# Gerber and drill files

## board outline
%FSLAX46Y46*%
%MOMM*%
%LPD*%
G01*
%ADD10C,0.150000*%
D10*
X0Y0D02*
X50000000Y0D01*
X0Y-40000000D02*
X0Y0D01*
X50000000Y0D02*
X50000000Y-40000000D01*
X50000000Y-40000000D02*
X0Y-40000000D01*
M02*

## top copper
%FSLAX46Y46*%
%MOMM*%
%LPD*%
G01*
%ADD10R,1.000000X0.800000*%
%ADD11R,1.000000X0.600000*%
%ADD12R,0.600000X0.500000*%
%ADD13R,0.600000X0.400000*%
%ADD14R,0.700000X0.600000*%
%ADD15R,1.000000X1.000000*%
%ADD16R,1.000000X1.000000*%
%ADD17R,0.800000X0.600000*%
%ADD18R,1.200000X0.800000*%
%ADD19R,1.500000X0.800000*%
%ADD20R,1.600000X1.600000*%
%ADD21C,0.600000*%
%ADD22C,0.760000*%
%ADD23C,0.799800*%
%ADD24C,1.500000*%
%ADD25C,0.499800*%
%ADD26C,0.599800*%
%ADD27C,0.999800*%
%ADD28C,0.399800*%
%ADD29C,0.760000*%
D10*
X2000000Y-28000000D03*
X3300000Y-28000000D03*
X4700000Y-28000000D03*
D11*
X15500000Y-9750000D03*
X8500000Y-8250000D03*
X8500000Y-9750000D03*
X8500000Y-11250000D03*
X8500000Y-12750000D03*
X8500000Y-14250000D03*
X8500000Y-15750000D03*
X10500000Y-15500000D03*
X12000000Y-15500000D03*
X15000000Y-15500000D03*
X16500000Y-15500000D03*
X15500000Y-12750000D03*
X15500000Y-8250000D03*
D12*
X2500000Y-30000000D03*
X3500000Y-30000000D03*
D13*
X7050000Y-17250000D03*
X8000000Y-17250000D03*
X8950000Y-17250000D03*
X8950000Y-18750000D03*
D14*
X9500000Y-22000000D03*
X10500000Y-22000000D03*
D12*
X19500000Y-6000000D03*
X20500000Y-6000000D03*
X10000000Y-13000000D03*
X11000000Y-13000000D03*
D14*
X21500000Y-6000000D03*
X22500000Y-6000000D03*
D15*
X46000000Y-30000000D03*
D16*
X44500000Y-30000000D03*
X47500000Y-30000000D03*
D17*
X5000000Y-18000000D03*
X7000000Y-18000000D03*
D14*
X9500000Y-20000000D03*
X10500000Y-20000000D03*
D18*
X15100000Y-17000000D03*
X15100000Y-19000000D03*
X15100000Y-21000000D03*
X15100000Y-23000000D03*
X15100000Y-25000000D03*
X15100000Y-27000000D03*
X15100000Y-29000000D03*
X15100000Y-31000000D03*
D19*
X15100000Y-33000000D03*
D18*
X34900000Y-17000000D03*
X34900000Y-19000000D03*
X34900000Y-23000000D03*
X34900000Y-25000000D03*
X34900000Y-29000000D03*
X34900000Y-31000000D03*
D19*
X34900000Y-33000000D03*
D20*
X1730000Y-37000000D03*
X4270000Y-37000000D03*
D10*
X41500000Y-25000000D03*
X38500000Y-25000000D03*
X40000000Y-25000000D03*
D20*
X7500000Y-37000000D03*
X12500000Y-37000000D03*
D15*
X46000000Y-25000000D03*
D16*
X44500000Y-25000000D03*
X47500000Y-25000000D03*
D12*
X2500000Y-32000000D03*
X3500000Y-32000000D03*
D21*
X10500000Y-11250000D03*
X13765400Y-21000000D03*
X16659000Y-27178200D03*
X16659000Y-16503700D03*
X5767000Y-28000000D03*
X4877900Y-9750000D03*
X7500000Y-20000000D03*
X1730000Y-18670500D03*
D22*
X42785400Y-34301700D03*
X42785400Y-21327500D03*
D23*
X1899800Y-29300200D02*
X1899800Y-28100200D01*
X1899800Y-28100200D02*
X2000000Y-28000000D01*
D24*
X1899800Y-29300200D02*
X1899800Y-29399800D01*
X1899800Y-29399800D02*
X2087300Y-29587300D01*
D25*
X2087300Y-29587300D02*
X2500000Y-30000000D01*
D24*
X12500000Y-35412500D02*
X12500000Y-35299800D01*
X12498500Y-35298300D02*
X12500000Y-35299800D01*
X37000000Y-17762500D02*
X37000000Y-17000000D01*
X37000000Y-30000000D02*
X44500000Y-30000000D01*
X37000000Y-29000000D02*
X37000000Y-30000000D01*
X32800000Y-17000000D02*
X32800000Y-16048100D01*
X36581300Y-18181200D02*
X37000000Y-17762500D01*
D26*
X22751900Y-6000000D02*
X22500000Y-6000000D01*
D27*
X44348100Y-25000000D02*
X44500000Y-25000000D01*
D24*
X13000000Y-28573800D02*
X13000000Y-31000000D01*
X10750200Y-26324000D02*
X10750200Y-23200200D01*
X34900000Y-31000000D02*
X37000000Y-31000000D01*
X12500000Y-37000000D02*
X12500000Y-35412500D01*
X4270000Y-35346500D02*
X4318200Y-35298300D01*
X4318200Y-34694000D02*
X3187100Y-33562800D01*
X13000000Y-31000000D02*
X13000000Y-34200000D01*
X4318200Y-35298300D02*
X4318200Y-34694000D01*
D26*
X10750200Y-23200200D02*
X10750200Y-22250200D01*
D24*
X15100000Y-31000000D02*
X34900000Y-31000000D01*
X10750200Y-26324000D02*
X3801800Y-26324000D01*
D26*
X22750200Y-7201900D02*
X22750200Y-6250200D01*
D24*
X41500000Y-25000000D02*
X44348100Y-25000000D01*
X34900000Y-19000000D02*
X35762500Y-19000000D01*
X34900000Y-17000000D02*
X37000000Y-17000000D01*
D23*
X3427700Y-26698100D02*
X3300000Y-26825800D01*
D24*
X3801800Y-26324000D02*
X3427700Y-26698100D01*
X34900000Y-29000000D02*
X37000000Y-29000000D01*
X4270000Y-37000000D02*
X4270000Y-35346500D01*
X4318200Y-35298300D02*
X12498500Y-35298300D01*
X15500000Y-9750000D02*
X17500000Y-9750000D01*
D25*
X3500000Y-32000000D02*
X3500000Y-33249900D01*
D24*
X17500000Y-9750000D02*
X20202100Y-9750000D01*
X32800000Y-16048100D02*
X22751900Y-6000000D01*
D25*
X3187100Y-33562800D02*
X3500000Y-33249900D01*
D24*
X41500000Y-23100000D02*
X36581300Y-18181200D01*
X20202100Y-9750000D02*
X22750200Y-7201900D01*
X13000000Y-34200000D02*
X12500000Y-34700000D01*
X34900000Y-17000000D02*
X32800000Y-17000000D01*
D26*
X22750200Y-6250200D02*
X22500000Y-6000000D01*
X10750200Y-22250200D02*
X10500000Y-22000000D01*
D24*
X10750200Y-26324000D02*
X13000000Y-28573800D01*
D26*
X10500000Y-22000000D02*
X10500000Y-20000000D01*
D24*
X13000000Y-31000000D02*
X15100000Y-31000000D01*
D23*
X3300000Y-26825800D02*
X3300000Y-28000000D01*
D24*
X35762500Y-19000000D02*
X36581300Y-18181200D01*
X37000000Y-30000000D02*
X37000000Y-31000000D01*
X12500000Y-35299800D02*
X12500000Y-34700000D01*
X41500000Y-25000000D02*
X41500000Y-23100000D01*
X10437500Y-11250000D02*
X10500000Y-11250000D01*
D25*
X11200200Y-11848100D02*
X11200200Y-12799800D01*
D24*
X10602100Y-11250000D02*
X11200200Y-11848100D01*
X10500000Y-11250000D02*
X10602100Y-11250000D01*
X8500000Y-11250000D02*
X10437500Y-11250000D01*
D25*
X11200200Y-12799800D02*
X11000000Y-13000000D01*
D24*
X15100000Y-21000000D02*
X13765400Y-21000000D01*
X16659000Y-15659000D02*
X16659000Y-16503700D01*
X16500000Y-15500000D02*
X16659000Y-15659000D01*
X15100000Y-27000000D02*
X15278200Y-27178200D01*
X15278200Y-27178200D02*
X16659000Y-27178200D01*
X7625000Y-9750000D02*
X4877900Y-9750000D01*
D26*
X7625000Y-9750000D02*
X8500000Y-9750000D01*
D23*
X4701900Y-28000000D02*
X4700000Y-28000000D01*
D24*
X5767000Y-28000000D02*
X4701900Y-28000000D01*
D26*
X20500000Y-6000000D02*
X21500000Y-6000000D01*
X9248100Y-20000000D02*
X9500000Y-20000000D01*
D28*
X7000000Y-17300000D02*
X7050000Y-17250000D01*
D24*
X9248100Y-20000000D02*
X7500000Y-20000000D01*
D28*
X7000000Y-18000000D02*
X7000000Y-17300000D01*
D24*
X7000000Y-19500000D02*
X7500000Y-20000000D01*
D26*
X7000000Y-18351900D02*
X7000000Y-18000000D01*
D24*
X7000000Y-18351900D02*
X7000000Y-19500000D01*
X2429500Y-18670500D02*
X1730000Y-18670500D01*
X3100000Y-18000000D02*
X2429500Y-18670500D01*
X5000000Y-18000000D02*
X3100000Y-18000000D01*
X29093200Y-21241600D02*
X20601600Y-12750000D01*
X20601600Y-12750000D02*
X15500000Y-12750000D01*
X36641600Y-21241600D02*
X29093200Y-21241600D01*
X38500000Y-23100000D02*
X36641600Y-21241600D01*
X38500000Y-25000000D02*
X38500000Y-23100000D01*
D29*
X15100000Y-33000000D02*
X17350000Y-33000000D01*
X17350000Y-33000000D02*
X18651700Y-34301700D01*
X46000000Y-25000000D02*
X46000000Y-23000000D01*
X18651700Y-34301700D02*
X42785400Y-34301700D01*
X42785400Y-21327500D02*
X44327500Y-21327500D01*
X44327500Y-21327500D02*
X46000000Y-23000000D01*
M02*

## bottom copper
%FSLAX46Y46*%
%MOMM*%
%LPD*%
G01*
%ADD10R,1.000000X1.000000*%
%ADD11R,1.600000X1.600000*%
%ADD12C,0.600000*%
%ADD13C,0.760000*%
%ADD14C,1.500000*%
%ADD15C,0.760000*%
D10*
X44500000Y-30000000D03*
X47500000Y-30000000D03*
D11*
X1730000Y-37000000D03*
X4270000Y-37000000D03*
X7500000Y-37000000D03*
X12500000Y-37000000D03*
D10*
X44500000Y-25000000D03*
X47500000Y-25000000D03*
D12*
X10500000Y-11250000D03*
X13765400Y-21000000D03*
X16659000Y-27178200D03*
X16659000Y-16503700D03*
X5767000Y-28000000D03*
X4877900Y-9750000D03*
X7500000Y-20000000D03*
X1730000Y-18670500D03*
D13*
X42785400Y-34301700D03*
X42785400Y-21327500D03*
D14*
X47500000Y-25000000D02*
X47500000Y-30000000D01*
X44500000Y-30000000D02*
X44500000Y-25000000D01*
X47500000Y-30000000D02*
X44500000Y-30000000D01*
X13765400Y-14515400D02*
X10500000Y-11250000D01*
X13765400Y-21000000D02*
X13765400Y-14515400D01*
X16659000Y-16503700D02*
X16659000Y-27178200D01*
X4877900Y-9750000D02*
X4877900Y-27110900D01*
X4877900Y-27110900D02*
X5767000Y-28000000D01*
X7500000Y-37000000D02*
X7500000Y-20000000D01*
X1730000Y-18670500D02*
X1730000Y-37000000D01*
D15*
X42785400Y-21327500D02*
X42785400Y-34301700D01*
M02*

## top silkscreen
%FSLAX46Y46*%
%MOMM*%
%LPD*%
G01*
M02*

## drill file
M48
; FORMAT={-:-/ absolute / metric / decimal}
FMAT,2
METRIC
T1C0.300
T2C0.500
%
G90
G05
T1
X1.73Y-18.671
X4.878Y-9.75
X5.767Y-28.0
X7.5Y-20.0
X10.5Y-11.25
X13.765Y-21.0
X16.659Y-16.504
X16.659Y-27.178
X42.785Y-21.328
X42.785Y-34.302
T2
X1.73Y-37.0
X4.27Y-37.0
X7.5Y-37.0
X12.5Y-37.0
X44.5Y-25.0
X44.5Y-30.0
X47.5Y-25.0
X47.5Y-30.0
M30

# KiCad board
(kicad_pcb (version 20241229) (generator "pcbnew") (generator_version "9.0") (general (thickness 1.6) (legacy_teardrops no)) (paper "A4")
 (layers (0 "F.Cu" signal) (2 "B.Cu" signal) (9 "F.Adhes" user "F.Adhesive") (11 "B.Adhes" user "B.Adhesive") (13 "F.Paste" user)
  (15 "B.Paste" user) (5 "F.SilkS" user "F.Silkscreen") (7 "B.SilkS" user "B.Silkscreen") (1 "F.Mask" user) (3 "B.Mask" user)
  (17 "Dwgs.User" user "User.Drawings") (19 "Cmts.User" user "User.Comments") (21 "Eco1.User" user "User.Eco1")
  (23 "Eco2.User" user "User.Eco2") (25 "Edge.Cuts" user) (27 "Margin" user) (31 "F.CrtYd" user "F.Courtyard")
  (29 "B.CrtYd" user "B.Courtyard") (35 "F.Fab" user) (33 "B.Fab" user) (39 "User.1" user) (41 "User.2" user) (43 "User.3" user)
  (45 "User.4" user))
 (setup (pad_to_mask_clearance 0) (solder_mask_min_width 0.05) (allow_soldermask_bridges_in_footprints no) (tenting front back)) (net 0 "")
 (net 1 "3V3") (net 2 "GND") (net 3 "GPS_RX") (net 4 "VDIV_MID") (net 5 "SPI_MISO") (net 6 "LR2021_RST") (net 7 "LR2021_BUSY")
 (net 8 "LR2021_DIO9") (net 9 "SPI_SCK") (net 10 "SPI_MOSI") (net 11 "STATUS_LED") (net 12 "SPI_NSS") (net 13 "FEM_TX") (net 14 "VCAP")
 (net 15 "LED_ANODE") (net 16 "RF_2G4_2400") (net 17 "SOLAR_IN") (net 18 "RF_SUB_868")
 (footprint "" (layer "F.Cu") (at 4 28)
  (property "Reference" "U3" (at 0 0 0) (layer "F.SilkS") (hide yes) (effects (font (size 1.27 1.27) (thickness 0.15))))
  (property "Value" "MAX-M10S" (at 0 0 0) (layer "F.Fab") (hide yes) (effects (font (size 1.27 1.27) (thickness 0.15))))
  (pad "1" smd rect (at -2 0) (size 1 0.8) (layers "F.Cu" "F.Mask") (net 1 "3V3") (thermal_bridge_angle 45))
  (pad "2" smd rect (at -0.7 0) (size 1 0.8) (layers "F.Cu" "F.Mask") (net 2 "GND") (thermal_bridge_angle 45))
  (pad "3" smd rect (at 0.7 0) (size 1 0.8) (layers "F.Cu" "F.Mask") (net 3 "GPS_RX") (thermal_bridge_angle 45)))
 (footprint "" (layer "F.Cu") (at 12 12)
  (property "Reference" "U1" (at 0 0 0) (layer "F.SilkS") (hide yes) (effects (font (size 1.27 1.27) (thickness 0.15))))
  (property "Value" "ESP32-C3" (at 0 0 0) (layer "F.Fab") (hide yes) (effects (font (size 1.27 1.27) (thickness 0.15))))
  (pad "GND" smd rect (at 3.5 -2.25) (size 1 0.6) (layers "F.Cu" "F.Mask") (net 2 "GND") (thermal_bridge_angle 45))
  (pad "GPIO0" smd rect (at -3.5 -3.75) (size 1 0.6) (layers "F.Cu" "F.Mask") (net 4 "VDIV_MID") (thermal_bridge_angle 45))
  (pad "GPIO1" smd rect (at -3.5 -2.25) (size 1 0.6) (layers "F.Cu" "F.Mask") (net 3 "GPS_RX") (thermal_bridge_angle 45))
  (pad "GPIO2" smd rect (at -3.5 -0.75) (size 1 0.6) (layers "F.Cu" "F.Mask") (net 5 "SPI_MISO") (thermal_bridge_angle 45))
  (pad "GPIO3" smd rect (at -3.5 0.75) (size 1 0.6) (layers "F.Cu" "F.Mask") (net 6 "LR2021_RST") (thermal_bridge_angle 45))
  (pad "GPIO4" smd rect (at -3.5 2.25) (size 1 0.6) (layers "F.Cu" "F.Mask") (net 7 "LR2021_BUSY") (thermal_bridge_angle 45))
  (pad "GPIO5" smd rect (at -3.5 3.75) (size 1 0.6) (layers "F.Cu" "F.Mask") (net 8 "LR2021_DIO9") (thermal_bridge_angle 45))
  (pad "GPIO6" smd rect (at -1.5 3.5) (size 1 0.6) (layers "F.Cu" "F.Mask") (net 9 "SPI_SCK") (thermal_bridge_angle 45))
  (pad "GPIO7" smd rect (at 0 3.5) (size 1 0.6) (layers "F.Cu" "F.Mask") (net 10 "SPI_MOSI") (thermal_bridge_angle 45))
  (pad "GPIO9" smd rect (at 3 3.5) (size 1 0.6) (layers "F.Cu" "F.Mask") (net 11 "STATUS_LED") (thermal_bridge_angle 45))
  (pad "GPIO10" smd rect (at 4.5 3.5) (size 1 0.6) (layers "F.Cu" "F.Mask") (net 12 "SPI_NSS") (thermal_bridge_angle 45))
  (pad "GPIO19" smd rect (at 3.5 0.75) (size 1 0.6) (layers "F.Cu" "F.Mask") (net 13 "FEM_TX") (thermal_bridge_angle 45))
  (pad "VCC" smd rect (at 3.5 -3.75) (size 1 0.6) (layers "F.Cu" "F.Mask") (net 1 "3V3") (thermal_bridge_angle 45)))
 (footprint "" (layer "F.Cu") (at 3 30)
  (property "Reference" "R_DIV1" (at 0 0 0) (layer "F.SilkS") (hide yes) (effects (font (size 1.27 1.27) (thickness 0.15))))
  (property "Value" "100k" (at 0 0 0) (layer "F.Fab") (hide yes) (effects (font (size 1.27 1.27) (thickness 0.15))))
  (pad "1" smd rect (at -0.5 0) (size 0.6 0.5) (layers "F.Cu" "F.Mask") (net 1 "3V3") (thermal_bridge_angle 45))
  (pad "2" smd rect (at 0.5 0) (size 0.6 0.5) (layers "F.Cu" "F.Mask") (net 4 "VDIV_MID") (thermal_bridge_angle 45)))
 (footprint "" (layer "F.Cu") (at 8 18)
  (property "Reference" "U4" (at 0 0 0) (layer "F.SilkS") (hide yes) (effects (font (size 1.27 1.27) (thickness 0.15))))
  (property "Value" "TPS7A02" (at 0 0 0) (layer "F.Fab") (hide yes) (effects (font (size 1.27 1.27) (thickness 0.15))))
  (pad "1" smd rect (at -0.95 -0.75) (size 0.6 0.4) (layers "F.Cu" "F.Mask") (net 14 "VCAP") (thermal_bridge_angle 45))
  (pad "2" smd rect (at 0 -0.75) (size 0.6 0.4) (layers "F.Cu" "F.Mask") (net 2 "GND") (thermal_bridge_angle 45))
  (pad "3" smd rect (at 0.95 -0.75) (size 0.6 0.4) (layers "F.Cu" "F.Mask") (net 14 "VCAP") (thermal_bridge_angle 45))
  (pad "4" smd rect (at 0.95 0.75) (size 0.6 0.4) (layers "F.Cu" "F.Mask") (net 1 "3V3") (thermal_bridge_angle 45)))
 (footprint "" (layer "F.Cu") (at 10 22)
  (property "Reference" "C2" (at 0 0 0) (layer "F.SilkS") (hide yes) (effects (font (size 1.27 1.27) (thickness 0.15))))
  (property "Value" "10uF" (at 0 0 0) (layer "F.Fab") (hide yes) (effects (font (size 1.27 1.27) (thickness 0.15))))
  (pad "1" smd rect (at -0.5 0) (size 0.7 0.6) (layers "F.Cu" "F.Mask") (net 1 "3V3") (thermal_bridge_angle 45))
  (pad "2" smd rect (at 0.5 0) (size 0.7 0.6) (layers "F.Cu" "F.Mask") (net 2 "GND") (thermal_bridge_angle 45)))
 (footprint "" (layer "F.Cu") (at 20 6)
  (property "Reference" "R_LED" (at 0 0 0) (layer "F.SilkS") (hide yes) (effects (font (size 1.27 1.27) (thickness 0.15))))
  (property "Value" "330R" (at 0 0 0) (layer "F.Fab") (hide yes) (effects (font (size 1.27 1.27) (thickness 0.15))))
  (pad "1" smd rect (at -0.5 0) (size 0.6 0.5) (layers "F.Cu" "F.Mask") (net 11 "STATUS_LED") (thermal_bridge_angle 45))
  (pad "2" smd rect (at 0.5 0) (size 0.6 0.5) (layers "F.Cu" "F.Mask") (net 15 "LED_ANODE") (thermal_bridge_angle 45)))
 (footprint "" (layer "F.Cu") (at 10.5 13)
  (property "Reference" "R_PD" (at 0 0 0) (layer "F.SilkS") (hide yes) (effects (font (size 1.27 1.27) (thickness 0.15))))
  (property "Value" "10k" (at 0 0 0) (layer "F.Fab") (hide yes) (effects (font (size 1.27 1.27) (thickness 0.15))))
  (pad "1" smd rect (at -0.5 0) (size 0.6 0.5) (layers "F.Cu" "F.Mask") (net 2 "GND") (thermal_bridge_angle 45))
  (pad "2" smd rect (at 0.5 0) (size 0.6 0.5) (layers "F.Cu" "F.Mask") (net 5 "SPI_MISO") (thermal_bridge_angle 45)))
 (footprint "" (layer "F.Cu") (at 22 6)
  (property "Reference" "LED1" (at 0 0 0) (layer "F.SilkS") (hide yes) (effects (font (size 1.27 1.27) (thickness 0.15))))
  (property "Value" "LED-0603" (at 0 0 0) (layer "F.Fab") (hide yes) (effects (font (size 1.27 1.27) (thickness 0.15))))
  (pad "A" smd rect (at -0.5 0) (size 0.7 0.6) (layers "F.Cu" "F.Mask") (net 15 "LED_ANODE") (thermal_bridge_angle 45))
  (pad "K" smd rect (at 0.5 0) (size 0.7 0.6) (layers "F.Cu" "F.Mask") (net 2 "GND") (thermal_bridge_angle 45)))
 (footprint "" (layer "F.Cu") (at 46 30)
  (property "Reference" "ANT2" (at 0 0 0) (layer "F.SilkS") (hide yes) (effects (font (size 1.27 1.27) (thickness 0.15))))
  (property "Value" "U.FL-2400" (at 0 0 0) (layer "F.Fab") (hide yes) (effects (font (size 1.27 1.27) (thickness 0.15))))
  (pad "1" smd rect (at 0 0) (size 1 1) (layers "F.Cu" "F.Mask") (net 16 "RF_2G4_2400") (thermal_bridge_angle 45))
  (pad "2" thru_hole rect (at -1.5 0) (size 1 1) (drill 0.5) (layers "*.Cu" "*.Mask") (remove_unused_layers no) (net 2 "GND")
   (thermal_bridge_angle 45))
  (pad "3" thru_hole rect (at 1.5 0) (size 1 1) (drill 0.5) (layers "*.Cu" "*.Mask") (remove_unused_layers no) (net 2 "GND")
   (thermal_bridge_angle 45)))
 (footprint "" (layer "F.Cu") (at 6 18)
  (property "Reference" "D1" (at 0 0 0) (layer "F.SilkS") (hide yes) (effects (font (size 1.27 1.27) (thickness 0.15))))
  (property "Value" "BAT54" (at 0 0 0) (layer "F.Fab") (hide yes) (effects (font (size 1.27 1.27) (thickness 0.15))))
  (pad "A" smd rect (at -1 0) (size 0.8 0.6) (layers "F.Cu" "F.Mask") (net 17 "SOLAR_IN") (thermal_bridge_angle 45))
  (pad "K" smd rect (at 1 0) (size 0.8 0.6) (layers "F.Cu" "F.Mask") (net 14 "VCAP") (thermal_bridge_angle 45)))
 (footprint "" (layer "F.Cu") (at 10 20)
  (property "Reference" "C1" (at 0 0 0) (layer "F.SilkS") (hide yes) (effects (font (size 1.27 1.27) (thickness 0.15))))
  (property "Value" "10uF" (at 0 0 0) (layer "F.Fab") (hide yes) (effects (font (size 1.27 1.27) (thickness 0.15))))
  (pad "1" smd rect (at -0.5 0) (size 0.7 0.6) (layers "F.Cu" "F.Mask") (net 14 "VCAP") (thermal_bridge_angle 45))
  (pad "2" smd rect (at 0.5 0) (size 0.7 0.6) (layers "F.Cu" "F.Mask") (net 2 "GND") (thermal_bridge_angle 45)))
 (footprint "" (layer "F.Cu") (at 25 25)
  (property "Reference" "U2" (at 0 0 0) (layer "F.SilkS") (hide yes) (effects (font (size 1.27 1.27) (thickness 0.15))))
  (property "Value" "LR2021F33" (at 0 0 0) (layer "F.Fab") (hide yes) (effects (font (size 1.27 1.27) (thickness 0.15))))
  (pad "1" smd rect (at -9.9 -8) (size 1.2 0.8) (layers "F.Cu" "F.Mask") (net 1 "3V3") (thermal_bridge_angle 45))
  (pad "2" smd rect (at -9.9 -6) (size 1.2 0.8) (layers "F.Cu" "F.Mask") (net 2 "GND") (thermal_bridge_angle 45))
  (pad "3" smd rect (at -9.9 -4) (size 1.2 0.8) (layers "F.Cu" "F.Mask") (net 5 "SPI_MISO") (thermal_bridge_angle 45))
  (pad "4" smd rect (at -9.9 -2) (size 1.2 0.8) (layers "F.Cu" "F.Mask") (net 10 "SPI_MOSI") (thermal_bridge_angle 45))
  (pad "5" smd rect (at -9.9 0) (size 1.2 0.8) (layers "F.Cu" "F.Mask") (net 9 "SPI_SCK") (thermal_bridge_angle 45))
  (pad "6" smd rect (at -9.9 2) (size 1.2 0.8) (layers "F.Cu" "F.Mask") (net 12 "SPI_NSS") (thermal_bridge_angle 45))
  (pad "7" smd rect (at -9.9 4) (size 1.2 0.8) (layers "F.Cu" "F.Mask") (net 7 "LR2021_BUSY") (thermal_bridge_angle 45))
  (pad "8" smd rect (at -9.9 6) (size 1.2 0.8) (layers "F.Cu" "F.Mask") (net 2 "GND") (thermal_bridge_angle 45))
  (pad "9" smd rect (at -9.9 8) (size 1.5 0.8) (layers "F.Cu" "F.Mask") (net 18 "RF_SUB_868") (thermal_bridge_angle 45))
  (pad "10" smd rect (at 9.9 -8) (size 1.2 0.8) (layers "F.Cu" "F.Mask") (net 2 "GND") (thermal_bridge_angle 45))
  (pad "11" smd rect (at 9.9 -6) (size 1.2 0.8) (layers "F.Cu" "F.Mask") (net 2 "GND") (thermal_bridge_angle 45))
  (pad "13" smd rect (at 9.9 -2) (size 1.2 0.8) (layers "F.Cu" "F.Mask") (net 8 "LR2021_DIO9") (thermal_bridge_angle 45))
  (pad "14" smd rect (at 9.9 0) (size 1.2 0.8) (layers "F.Cu" "F.Mask") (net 6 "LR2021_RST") (thermal_bridge_angle 45))
  (pad "16" smd rect (at 9.9 4) (size 1.2 0.8) (layers "F.Cu" "F.Mask") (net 2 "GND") (thermal_bridge_angle 45))
  (pad "17" smd rect (at 9.9 6) (size 1.2 0.8) (layers "F.Cu" "F.Mask") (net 2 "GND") (thermal_bridge_angle 45))
  (pad "18" smd rect (at 9.9 8) (size 1.5 0.8) (layers "F.Cu" "F.Mask") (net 16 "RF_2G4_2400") (thermal_bridge_angle 45)))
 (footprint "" (layer "F.Cu") (at 3 37)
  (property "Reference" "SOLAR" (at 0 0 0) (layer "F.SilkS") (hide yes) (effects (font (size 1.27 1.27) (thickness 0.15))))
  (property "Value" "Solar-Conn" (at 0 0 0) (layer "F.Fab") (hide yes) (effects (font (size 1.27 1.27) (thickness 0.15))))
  (pad "1" thru_hole rect (at -1.27 0) (size 1.6 1.6) (drill 0.5) (layers "*.Cu" "*.Mask") (remove_unused_layers no) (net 17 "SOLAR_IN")
   (thermal_bridge_angle 45))
  (pad "2" thru_hole rect (at 1.27 0) (size 1.6 1.6) (drill 0.5) (layers "*.Cu" "*.Mask") (remove_unused_layers no) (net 2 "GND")
   (thermal_bridge_angle 45)))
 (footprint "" (layer "F.Cu") (at 40 25)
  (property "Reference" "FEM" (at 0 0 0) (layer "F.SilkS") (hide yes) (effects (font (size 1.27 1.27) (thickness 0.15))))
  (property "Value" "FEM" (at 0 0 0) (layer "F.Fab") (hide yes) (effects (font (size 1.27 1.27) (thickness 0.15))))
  (pad "GND" smd rect (at 1.5 0) (size 1 0.8) (layers "F.Cu" "F.Mask") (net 2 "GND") (thermal_bridge_angle 45))
  (pad "TX" smd rect (at -1.5 0) (size 1 0.8) (layers "F.Cu" "F.Mask") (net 13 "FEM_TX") (thermal_bridge_angle 45))
  (pad "VCC" smd rect (at 0 0) (size 1 0.8) (layers "F.Cu" "F.Mask") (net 1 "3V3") (thermal_bridge_angle 45)))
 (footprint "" (layer "F.Cu") (at 10 37)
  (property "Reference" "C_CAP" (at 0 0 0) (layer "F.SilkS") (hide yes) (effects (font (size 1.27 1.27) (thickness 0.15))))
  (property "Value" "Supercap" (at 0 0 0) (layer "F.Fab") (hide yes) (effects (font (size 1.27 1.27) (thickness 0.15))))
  (pad "1" thru_hole rect (at -2.5 0) (size 1.6 1.6) (drill 0.5) (layers "*.Cu" "*.Mask") (remove_unused_layers no) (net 14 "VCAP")
   (thermal_bridge_angle 45))
  (pad "2" thru_hole rect (at 2.5 0) (size 1.6 1.6) (drill 0.5) (layers "*.Cu" "*.Mask") (remove_unused_layers no) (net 2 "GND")
   (thermal_bridge_angle 45)))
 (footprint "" (layer "F.Cu") (at 46 25)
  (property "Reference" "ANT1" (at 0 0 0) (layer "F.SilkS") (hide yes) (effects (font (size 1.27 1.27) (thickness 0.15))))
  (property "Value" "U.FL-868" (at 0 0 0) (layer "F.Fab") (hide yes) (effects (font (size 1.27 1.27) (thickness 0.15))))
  (pad "1" smd rect (at 0 0) (size 1 1) (layers "F.Cu" "F.Mask") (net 18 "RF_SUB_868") (thermal_bridge_angle 45))
  (pad "2" thru_hole rect (at -1.5 0) (size 1 1) (drill 0.5) (layers "*.Cu" "*.Mask") (remove_unused_layers no) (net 2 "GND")
   (thermal_bridge_angle 45))
  (pad "3" thru_hole rect (at 1.5 0) (size 1 1) (drill 0.5) (layers "*.Cu" "*.Mask") (remove_unused_layers no) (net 2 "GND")
   (thermal_bridge_angle 45)))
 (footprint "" (layer "F.Cu") (at 3 32)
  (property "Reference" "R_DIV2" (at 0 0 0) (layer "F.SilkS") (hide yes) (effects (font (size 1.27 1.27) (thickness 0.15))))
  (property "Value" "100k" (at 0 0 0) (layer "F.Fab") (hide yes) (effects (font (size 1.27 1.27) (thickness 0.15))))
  (pad "1" smd rect (at -0.5 0) (size 0.6 0.5) (layers "F.Cu" "F.Mask") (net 4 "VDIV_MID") (thermal_bridge_angle 45))
  (pad "2" smd rect (at 0.5 0) (size 0.6 0.5) (layers "F.Cu" "F.Mask") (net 2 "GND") (thermal_bridge_angle 45)))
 (gr_line (start 0 0) (end 50 0) (stroke (width 0.15) (type default)) (layer "Edge.Cuts"))
 (gr_line (start 0 40) (end 0 0) (stroke (width 0.15) (type default)) (layer "Edge.Cuts"))
 (gr_line (start 50 0) (end 50 40) (stroke (width 0.15) (type default)) (layer "Edge.Cuts"))
 (gr_line (start 50 40) (end 0 40) (stroke (width 0.15) (type default)) (layer "Edge.Cuts"))
 (segment (start 1.8998 29.3002) (end 1.8998 28.1002) (width 0.7998) (layer "F.Cu") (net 1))
 (segment (start 1.8998 28.1002) (end 2 28) (width 0.7998) (layer "F.Cu") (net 1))
 (segment (start 1.8998 29.3002) (end 1.8998 29.3998) (width 1.5) (layer "F.Cu") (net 1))
 (segment (start 1.8998 29.3998) (end 2.0873 29.5873) (width 1.5) (layer "F.Cu") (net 1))
 (segment (start 2.0873 29.5873) (end 2.5 30) (width 0.4998) (layer "F.Cu") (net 1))
 (segment (start 12.5 35.4125) (end 12.5 35.2998) (width 1.5) (layer "F.Cu") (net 2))
 (segment (start 12.4985 35.2983) (end 12.5 35.2998) (width 1.5) (layer "F.Cu") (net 2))
 (segment (start 37 17.7625) (end 37 17) (width 1.5) (layer "F.Cu") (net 2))
 (segment (start 37 30) (end 44.5 30) (width 1.5) (layer "F.Cu") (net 2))
 (segment (start 37 29) (end 37 30) (width 1.5) (layer "F.Cu") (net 2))
 (segment (start 32.8 17) (end 32.8 16.0481) (width 1.5) (layer "F.Cu") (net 2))
 (segment (start 36.5813 18.1812) (end 37 17.7625) (width 1.5) (layer "F.Cu") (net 2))
 (segment (start 22.7519 6) (end 22.5 6) (width 0.5998) (layer "F.Cu") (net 2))
 (segment (start 44.3481 25) (end 44.5 25) (width 0.9998) (layer "F.Cu") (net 2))
 (segment (start 13 28.5738) (end 13 31) (width 1.5) (layer "F.Cu") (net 2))
 (segment (start 10.7502 26.324) (end 10.7502 23.2002) (width 1.5) (layer "F.Cu") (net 2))
 (segment (start 34.9 31) (end 37 31) (width 1.5) (layer "F.Cu") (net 2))
 (segment (start 12.5 37) (end 12.5 35.4125) (width 1.5) (layer "F.Cu") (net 2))
 (segment (start 4.27 35.3465) (end 4.3182 35.2983) (width 1.5) (layer "F.Cu") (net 2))
 (segment (start 4.3182 34.694) (end 3.1871 33.5628) (width 1.5) (layer "F.Cu") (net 2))
 (segment (start 13 31) (end 13 34.2) (width 1.5) (layer "F.Cu") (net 2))
 (segment (start 4.3182 35.2983) (end 4.3182 34.694) (width 1.5) (layer "F.Cu") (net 2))
 (segment (start 10.7502 23.2002) (end 10.7502 22.2502) (width 0.5998) (layer "F.Cu") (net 2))
 (segment (start 15.1 31) (end 34.9 31) (width 1.5) (layer "F.Cu") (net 2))
 (segment (start 10.7502 26.324) (end 3.8018 26.324) (width 1.5) (layer "F.Cu") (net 2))
 (segment (start 22.7502 7.2019) (end 22.7502 6.2502) (width 0.5998) (layer "F.Cu") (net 2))
 (segment (start 41.5 25) (end 44.3481 25) (width 1.5) (layer "F.Cu") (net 2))
 (segment (start 34.9 19) (end 35.7625 19) (width 1.5) (layer "F.Cu") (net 2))
 (segment (start 34.9 17) (end 37 17) (width 1.5) (layer "F.Cu") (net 2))
 (segment (start 3.4277 26.6981) (end 3.3 26.8258) (width 0.7998) (layer "F.Cu") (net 2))
 (segment (start 3.8018 26.324) (end 3.4277 26.6981) (width 1.5) (layer "F.Cu") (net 2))
 (segment (start 34.9 29) (end 37 29) (width 1.5) (layer "F.Cu") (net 2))
 (segment (start 4.27 37) (end 4.27 35.3465) (width 1.5) (layer "F.Cu") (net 2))
 (segment (start 4.3182 35.2983) (end 12.4985 35.2983) (width 1.5) (layer "F.Cu") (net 2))
 (segment (start 15.5 9.75) (end 17.5 9.75) (width 1.5) (layer "F.Cu") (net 2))
 (segment (start 3.5 32) (end 3.5 33.2499) (width 0.4998) (layer "F.Cu") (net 2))
 (segment (start 17.5 9.75) (end 20.2021 9.75) (width 1.5) (layer "F.Cu") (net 2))
 (segment (start 32.8 16.0481) (end 22.7519 6) (width 1.5) (layer "F.Cu") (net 2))
 (segment (start 3.1871 33.5628) (end 3.5 33.2499) (width 0.4998) (layer "F.Cu") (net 2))
 (segment (start 41.5 23.1) (end 36.5813 18.1812) (width 1.5) (layer "F.Cu") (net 2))
 (segment (start 20.2021 9.75) (end 22.7502 7.2019) (width 1.5) (layer "F.Cu") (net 2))
 (segment (start 13 34.2) (end 12.5 34.7) (width 1.5) (layer "F.Cu") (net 2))
 (segment (start 34.9 17) (end 32.8 17) (width 1.5) (layer "F.Cu") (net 2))
 (segment (start 22.7502 6.2502) (end 22.5 6) (width 0.5998) (layer "F.Cu") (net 2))
 (segment (start 10.7502 22.2502) (end 10.5 22) (width 0.5998) (layer "F.Cu") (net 2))
 (segment (start 10.7502 26.324) (end 13 28.5738) (width 1.5) (layer "F.Cu") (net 2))
 (segment (start 10.5 22) (end 10.5 20) (width 0.5998) (layer "F.Cu") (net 2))
 (segment (start 13 31) (end 15.1 31) (width 1.5) (layer "F.Cu") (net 2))
 (segment (start 3.3 26.8258) (end 3.3 28) (width 0.7998) (layer "F.Cu") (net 2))
 (segment (start 35.7625 19) (end 36.5813 18.1812) (width 1.5) (layer "F.Cu") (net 2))
 (segment (start 37 30) (end 37 31) (width 1.5) (layer "F.Cu") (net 2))
 (segment (start 12.5 35.2998) (end 12.5 34.7) (width 1.5) (layer "F.Cu") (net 2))
 (segment (start 41.5 25) (end 41.5 23.1) (width 1.5) (layer "F.Cu") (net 2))
 (segment (start 47.5 25) (end 47.5 30) (width 1.5) (layer "B.Cu") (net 2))
 (segment (start 44.5 30) (end 44.5 25) (width 1.5) (layer "B.Cu") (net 2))
 (segment (start 47.5 30) (end 44.5 30) (width 1.5) (layer "B.Cu") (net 2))
 (segment (start 10.4375 11.25) (end 10.5 11.25) (width 1.5) (layer "F.Cu") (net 5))
 (segment (start 11.2002 11.8481) (end 11.2002 12.7998) (width 0.4998) (layer "F.Cu") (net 5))
 (segment (start 10.6021 11.25) (end 11.2002 11.8481) (width 1.5) (layer "F.Cu") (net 5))
 (segment (start 10.5 11.25) (end 10.6021 11.25) (width 1.5) (layer "F.Cu") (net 5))
 (segment (start 8.5 11.25) (end 10.4375 11.25) (width 1.5) (layer "F.Cu") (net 5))
 (segment (start 11.2002 12.7998) (end 11 13) (width 0.4998) (layer "F.Cu") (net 5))
 (segment (start 15.1 21) (end 13.7654 21) (width 1.5) (layer "F.Cu") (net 5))
 (via (at 10.5 11.25) (size 0.6) (drill 0.3) (layers "F.Cu" "B.Cu") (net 5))
 (via (at 13.7654 21) (size 0.6) (drill 0.3) (layers "F.Cu" "B.Cu") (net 5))
 (segment (start 13.7654 14.5154) (end 10.5 11.25) (width 1.5) (layer "B.Cu") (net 5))
 (segment (start 13.7654 21) (end 13.7654 14.5154) (width 1.5) (layer "B.Cu") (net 5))
 (segment (start 16.659 15.659) (end 16.659 16.5037) (width 1.5) (layer "F.Cu") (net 12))
 (segment (start 16.5 15.5) (end 16.659 15.659) (width 1.5) (layer "F.Cu") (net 12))
 (segment (start 15.1 27) (end 15.2782 27.1782) (width 1.5) (layer "F.Cu") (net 12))
 (segment (start 15.2782 27.1782) (end 16.659 27.1782) (width 1.5) (layer "F.Cu") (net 12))
 (via (at 16.659 27.1782) (size 0.6) (drill 0.3) (layers "F.Cu" "B.Cu") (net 12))
 (via (at 16.659 16.5037) (size 0.6) (drill 0.3) (layers "F.Cu" "B.Cu") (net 12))
 (segment (start 16.659 16.5037) (end 16.659 27.1782) (width 1.5) (layer "B.Cu") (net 12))
 (segment (start 7.625 9.75) (end 4.8779 9.75) (width 1.5) (layer "F.Cu") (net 3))
 (segment (start 7.625 9.75) (end 8.5 9.75) (width 0.5998) (layer "F.Cu") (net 3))
 (segment (start 4.7019 28) (end 4.7 28) (width 0.7998) (layer "F.Cu") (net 3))
 (segment (start 5.767 28) (end 4.7019 28) (width 1.5) (layer "F.Cu") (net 3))
 (via (at 5.767 28) (size 0.6) (drill 0.3) (layers "F.Cu" "B.Cu") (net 3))
 (via (at 4.8779 9.75) (size 0.6) (drill 0.3) (layers "F.Cu" "B.Cu") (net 3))
 (segment (start 4.8779 9.75) (end 4.8779 27.1109) (width 1.5) (layer "B.Cu") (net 3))
 (segment (start 4.8779 27.1109) (end 5.767 28) (width 1.5) (layer "B.Cu") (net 3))
 (segment (start 20.5 6) (end 21.5 6) (width 0.5998) (layer "F.Cu") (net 15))
 (segment (start 9.2481 20) (end 9.5 20) (width 0.5998) (layer "F.Cu") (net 14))
 (segment (start 7 17.3) (end 7.05 17.25) (width 0.3998) (layer "F.Cu") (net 14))
 (segment (start 9.2481 20) (end 7.5 20) (width 1.5) (layer "F.Cu") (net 14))
 (segment (start 7 18) (end 7 17.3) (width 0.3998) (layer "F.Cu") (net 14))
 (segment (start 7 19.5) (end 7.5 20) (width 1.5) (layer "F.Cu") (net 14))
 (segment (start 7 18.3519) (end 7 18) (width 0.5998) (layer "F.Cu") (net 14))
 (segment (start 7 18.3519) (end 7 19.5) (width 1.5) (layer "F.Cu") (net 14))
 (via (at 7.5 20) (size 0.6) (drill 0.3) (layers "F.Cu" "B.Cu") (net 14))
 (segment (start 7.5 37) (end 7.5 20) (width 1.5) (layer "B.Cu") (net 14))
 (segment (start 2.4295 18.6705) (end 1.73 18.6705) (width 1.5) (layer "F.Cu") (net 17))
 (segment (start 3.1 18) (end 2.4295 18.6705) (width 1.5) (layer "F.Cu") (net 17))
 (segment (start 5 18) (end 3.1 18) (width 1.5) (layer "F.Cu") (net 17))
 (via (at 1.73 18.6705) (size 0.6) (drill 0.3) (layers "F.Cu" "B.Cu") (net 17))
 (segment (start 1.73 18.6705) (end 1.73 37) (width 1.5) (layer "B.Cu") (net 17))
 (segment (start 29.0932 21.2416) (end 20.6016 12.75) (width 1.5) (layer "F.Cu") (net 13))
 (segment (start 20.6016 12.75) (end 15.5 12.75) (width 1.5) (layer "F.Cu") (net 13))
 (segment (start 36.6416 21.2416) (end 29.0932 21.2416) (width 1.5) (layer "F.Cu") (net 13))
 (segment (start 38.5 23.1) (end 36.6416 21.2416) (width 1.5) (layer "F.Cu") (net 13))
 (segment (start 38.5 25) (end 38.5 23.1) (width 1.5) (layer "F.Cu") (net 13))
 (segment (start 15.1 33) (end 17.35 33) (width 0.76) (layer "F.Cu") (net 18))
 (segment (start 17.35 33) (end 18.6517 34.3017) (width 0.76) (layer "F.Cu") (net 18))
 (segment (start 46 25) (end 46 23) (width 0.76) (layer "F.Cu") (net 18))
 (segment (start 18.6517 34.3017) (end 42.7854 34.3017) (width 0.76) (layer "F.Cu") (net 18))
 (segment (start 42.7854 21.3275) (end 44.3275 21.3275) (width 0.76) (layer "F.Cu") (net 18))
 (segment (start 44.3275 21.3275) (end 46 23) (width 0.76) (layer "F.Cu") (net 18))
 (via (at 42.7854 34.3017) (size 0.76) (drill 0.3) (layers "F.Cu" "B.Cu") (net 18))
 (via (at 42.7854 21.3275) (size 0.76) (drill 0.3) (layers "F.Cu" "B.Cu") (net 18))
 (segment (start 42.7854 21.3275) (end 42.7854 34.3017) (width 0.76) (layer "B.Cu") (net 18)))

